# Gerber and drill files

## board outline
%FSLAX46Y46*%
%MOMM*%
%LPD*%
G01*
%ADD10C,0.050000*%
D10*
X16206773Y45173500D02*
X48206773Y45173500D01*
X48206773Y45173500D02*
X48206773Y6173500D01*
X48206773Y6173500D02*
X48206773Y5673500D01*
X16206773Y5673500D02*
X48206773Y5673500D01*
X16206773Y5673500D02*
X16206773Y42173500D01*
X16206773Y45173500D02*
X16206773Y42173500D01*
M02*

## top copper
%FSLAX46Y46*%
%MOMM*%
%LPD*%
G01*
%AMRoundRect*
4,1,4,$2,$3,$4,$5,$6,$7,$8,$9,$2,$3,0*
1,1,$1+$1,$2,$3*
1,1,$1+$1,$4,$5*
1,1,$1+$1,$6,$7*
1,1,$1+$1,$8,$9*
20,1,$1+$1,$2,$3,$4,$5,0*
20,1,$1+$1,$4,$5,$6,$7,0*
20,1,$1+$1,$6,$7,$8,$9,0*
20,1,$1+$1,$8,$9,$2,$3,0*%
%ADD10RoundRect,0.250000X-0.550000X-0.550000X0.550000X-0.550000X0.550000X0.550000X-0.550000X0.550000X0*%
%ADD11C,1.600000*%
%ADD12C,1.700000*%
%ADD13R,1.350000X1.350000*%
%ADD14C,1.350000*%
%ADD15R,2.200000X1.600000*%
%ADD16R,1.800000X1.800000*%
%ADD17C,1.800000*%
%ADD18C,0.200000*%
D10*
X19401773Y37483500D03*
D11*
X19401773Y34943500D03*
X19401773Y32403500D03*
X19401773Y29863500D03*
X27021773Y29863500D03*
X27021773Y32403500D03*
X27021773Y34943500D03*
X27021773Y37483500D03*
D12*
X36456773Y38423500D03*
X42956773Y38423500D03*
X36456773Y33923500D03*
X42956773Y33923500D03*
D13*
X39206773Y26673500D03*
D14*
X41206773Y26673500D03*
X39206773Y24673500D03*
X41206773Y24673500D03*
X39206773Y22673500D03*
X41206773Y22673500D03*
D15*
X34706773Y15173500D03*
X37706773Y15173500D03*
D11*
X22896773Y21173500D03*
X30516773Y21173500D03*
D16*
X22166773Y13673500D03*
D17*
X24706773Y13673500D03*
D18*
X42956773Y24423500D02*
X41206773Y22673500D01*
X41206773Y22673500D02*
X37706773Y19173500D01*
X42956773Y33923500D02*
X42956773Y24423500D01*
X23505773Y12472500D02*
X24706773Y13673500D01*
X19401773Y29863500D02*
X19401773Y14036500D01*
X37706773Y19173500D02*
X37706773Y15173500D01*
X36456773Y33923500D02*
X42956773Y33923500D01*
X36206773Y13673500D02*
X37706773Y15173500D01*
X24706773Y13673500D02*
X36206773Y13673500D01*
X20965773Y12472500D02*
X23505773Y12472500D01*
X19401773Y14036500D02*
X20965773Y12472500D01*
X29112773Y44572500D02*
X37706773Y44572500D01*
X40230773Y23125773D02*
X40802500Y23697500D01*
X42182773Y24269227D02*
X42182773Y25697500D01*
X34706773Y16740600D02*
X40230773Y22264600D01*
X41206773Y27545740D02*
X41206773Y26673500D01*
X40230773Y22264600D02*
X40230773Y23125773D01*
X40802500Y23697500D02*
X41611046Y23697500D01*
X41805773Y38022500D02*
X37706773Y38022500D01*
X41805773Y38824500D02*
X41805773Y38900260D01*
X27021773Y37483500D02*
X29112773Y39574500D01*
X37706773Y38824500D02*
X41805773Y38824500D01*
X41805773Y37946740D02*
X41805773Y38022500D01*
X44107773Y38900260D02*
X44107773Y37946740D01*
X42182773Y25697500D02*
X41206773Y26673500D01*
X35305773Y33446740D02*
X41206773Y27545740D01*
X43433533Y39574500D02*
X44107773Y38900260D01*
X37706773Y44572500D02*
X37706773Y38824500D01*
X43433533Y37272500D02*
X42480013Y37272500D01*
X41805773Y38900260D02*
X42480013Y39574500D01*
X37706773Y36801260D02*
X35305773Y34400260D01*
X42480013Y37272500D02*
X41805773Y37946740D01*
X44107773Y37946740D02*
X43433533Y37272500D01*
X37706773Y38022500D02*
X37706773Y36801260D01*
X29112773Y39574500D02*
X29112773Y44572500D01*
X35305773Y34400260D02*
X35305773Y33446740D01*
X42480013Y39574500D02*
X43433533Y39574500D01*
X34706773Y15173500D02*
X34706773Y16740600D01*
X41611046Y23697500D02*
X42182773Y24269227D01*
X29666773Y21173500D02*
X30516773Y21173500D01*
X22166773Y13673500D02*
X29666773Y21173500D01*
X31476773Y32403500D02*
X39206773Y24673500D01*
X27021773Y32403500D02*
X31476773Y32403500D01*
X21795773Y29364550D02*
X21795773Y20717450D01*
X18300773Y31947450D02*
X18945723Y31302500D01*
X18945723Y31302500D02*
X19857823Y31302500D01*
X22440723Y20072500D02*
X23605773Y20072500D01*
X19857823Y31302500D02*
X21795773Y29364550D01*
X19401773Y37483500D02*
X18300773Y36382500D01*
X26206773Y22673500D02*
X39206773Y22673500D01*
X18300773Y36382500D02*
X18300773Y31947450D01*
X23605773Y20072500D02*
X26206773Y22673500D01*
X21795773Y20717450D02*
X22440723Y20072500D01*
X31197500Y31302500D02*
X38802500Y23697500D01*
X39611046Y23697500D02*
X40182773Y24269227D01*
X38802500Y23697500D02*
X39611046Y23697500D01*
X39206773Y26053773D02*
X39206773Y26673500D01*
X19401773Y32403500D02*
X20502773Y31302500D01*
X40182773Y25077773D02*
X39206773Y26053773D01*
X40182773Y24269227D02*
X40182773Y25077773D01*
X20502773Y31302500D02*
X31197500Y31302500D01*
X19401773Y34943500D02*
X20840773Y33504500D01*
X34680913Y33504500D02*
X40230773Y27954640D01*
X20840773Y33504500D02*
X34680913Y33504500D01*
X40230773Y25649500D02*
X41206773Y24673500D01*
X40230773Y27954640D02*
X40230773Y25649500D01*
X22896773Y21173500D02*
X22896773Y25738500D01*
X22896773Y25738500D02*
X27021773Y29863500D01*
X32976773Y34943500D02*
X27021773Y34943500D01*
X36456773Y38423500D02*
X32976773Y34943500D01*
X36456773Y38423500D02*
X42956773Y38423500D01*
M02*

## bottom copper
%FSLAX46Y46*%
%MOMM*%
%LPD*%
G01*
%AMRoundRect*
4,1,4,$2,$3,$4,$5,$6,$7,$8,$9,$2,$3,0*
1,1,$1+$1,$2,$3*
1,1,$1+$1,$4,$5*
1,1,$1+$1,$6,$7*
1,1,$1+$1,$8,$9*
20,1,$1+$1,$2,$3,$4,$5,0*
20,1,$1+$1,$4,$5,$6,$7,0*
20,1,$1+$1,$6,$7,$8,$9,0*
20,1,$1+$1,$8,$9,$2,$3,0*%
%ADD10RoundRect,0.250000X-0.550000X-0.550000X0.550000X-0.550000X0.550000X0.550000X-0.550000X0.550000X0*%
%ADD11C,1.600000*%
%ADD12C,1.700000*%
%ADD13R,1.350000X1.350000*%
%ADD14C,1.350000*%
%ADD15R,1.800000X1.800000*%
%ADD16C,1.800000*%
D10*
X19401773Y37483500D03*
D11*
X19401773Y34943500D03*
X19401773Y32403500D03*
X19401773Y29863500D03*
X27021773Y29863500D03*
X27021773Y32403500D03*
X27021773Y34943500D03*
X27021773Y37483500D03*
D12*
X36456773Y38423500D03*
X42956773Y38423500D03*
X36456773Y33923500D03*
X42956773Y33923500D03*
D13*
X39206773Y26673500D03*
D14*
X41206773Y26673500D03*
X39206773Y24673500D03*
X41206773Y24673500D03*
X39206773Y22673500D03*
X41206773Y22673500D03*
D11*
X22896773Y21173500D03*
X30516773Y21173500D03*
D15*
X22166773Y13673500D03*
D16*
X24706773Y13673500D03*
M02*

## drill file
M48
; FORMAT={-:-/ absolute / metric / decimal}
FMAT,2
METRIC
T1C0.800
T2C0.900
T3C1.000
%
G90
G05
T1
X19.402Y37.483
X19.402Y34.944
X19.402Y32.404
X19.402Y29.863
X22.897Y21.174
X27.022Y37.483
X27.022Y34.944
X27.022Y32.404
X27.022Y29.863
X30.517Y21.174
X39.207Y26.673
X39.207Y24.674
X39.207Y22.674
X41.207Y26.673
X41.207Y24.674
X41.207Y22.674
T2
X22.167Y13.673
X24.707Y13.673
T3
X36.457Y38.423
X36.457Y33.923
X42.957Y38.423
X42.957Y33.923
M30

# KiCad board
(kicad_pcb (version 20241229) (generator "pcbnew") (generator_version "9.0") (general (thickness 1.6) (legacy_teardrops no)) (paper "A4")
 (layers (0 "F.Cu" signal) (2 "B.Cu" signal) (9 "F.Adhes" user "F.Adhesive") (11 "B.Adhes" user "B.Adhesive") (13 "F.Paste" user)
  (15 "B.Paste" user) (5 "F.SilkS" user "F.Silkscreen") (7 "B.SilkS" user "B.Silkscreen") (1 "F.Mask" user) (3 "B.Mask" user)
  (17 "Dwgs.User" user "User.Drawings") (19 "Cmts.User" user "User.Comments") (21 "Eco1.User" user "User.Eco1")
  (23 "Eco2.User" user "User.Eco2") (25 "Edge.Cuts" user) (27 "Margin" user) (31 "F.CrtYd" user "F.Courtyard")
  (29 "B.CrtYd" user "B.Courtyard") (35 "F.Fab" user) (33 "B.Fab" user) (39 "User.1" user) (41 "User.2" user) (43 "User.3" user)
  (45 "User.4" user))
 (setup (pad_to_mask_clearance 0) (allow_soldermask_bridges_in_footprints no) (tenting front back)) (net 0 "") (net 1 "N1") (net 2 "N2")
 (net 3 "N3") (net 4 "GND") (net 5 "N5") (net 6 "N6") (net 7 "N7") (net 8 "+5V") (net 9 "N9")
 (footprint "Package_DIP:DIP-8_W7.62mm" (layer "F.Cu") (at 19.401773 -37.4835)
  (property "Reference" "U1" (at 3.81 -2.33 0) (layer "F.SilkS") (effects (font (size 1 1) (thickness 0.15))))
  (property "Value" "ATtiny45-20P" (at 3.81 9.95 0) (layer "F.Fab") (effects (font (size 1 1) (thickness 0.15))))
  (pad "1" thru_hole roundrect (at 0 0) (size 1.6 1.6) (drill 0.8) (layers "*.Cu" "*.Mask") (remove_unused_layers no)
   (roundrect_rratio 0.15625) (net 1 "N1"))
  (pad "2" thru_hole circle (at 0 2.54) (size 1.6 1.6) (drill 0.8) (layers "*.Cu" "*.Mask") (remove_unused_layers no) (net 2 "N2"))
  (pad "3" thru_hole circle (at 0 5.08) (size 1.6 1.6) (drill 0.8) (layers "*.Cu" "*.Mask") (remove_unused_layers no) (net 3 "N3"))
  (pad "4" thru_hole circle (at 0 7.62) (size 1.6 1.6) (drill 0.8) (layers "*.Cu" "*.Mask") (remove_unused_layers no) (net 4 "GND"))
  (pad "5" thru_hole circle (at 7.62 7.62) (size 1.6 1.6) (drill 0.8) (layers "*.Cu" "*.Mask") (remove_unused_layers no) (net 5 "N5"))
  (pad "6" thru_hole circle (at 7.62 5.08) (size 1.6 1.6) (drill 0.8) (layers "*.Cu" "*.Mask") (remove_unused_layers no) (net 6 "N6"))
  (pad "7" thru_hole circle (at 7.62 2.54) (size 1.6 1.6) (drill 0.8) (layers "*.Cu" "*.Mask") (remove_unused_layers no) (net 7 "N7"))
  (pad "8" thru_hole circle (at 7.62 0) (size 1.6 1.6) (drill 0.8) (layers "*.Cu" "*.Mask") (remove_unused_layers no) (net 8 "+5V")))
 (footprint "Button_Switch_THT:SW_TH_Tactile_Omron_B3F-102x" (layer "F.Cu") (at 36.456773 -38.4235)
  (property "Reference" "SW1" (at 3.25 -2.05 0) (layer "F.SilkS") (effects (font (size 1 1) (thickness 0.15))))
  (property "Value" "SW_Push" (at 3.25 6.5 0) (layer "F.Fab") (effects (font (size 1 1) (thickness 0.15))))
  (pad "1" thru_hole circle (at 0 0) (size 1.7 1.7) (drill 1) (layers "*.Cu" "*.Mask") (remove_unused_layers no) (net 7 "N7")
   (thermal_bridge_angle 90))
  (pad "1" thru_hole circle (at 6.5 0) (size 1.7 1.7) (drill 1) (layers "*.Cu" "*.Mask") (remove_unused_layers no) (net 7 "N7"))
  (pad "2" thru_hole circle (at 0 4.5) (size 1.7 1.7) (drill 1) (layers "*.Cu" "*.Mask") (remove_unused_layers no) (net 4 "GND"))
  (pad "2" thru_hole circle (at 6.5 4.5) (size 1.7 1.7) (drill 1) (layers "*.Cu" "*.Mask") (remove_unused_layers no) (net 4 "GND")))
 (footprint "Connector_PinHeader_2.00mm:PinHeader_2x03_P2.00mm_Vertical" (layer "F.Cu") (at 39.206773 -26.6735)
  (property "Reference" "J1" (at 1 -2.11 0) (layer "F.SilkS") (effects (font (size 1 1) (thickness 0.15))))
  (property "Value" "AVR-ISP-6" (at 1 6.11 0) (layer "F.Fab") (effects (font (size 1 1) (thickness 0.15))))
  (pad "1" thru_hole rect (at 0 0) (size 1.35 1.35) (drill 0.8) (layers "*.Cu" "*.Mask") (remove_unused_layers no) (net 3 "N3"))
  (pad "2" thru_hole circle (at 2 0) (size 1.35 1.35) (drill 0.8) (layers "*.Cu" "*.Mask") (remove_unused_layers no) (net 8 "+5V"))
  (pad "3" thru_hole circle (at 0 2) (size 1.35 1.35) (drill 0.8) (layers "*.Cu" "*.Mask") (remove_unused_layers no) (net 6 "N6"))
  (pad "4" thru_hole circle (at 2 2) (size 1.35 1.35) (drill 0.8) (layers "*.Cu" "*.Mask") (remove_unused_layers no) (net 2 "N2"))
  (pad "5" thru_hole circle (at 0 4) (size 1.35 1.35) (drill 0.8) (layers "*.Cu" "*.Mask") (remove_unused_layers no) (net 1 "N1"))
  (pad "6" thru_hole circle (at 2 4) (size 1.35 1.35) (drill 0.8) (layers "*.Cu" "*.Mask") (remove_unused_layers no) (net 4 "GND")))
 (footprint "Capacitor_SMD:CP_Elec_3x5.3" (layer "F.Cu") (at 36.206773 -15.1735)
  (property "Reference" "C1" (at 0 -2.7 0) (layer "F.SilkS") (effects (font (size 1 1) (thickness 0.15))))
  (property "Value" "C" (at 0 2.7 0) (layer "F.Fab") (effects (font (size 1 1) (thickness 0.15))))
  (pad "1" smd rect (at -1.5 0) (size 2.2 1.6) (layers "F.Cu" "F.Mask" "F.Paste") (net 8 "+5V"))
  (pad "2" smd rect (at 1.5 0) (size 2.2 1.6) (layers "F.Cu" "F.Mask" "F.Paste") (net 4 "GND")))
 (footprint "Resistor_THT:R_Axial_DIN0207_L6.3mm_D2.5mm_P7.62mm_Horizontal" (layer "F.Cu") (at 22.896773 -21.1735)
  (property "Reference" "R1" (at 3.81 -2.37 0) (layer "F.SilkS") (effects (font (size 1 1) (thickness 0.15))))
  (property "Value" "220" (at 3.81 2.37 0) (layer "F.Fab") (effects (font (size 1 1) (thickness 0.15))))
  (pad "1" thru_hole circle (at 0 0) (size 1.6 1.6) (drill 0.8) (layers "*.Cu" "*.Mask") (remove_unused_layers no) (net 5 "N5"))
  (pad "2" thru_hole circle (at 7.62 0) (size 1.6 1.6) (drill 0.8) (layers "*.Cu" "*.Mask") (remove_unused_layers no) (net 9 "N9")))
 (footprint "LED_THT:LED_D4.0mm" (layer "F.Cu") (at 22.166773 -13.6735)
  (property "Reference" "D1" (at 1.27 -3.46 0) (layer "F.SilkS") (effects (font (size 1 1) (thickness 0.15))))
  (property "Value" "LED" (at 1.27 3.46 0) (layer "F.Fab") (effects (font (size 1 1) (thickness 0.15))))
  (pad "1" thru_hole rect (at 0 0) (size 1.8 1.8) (drill 0.9) (layers "*.Cu" "*.Mask") (remove_unused_layers no) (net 9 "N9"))
  (pad "2" thru_hole circle (at 2.54 0) (size 1.8 1.8) (drill 0.9) (layers "*.Cu" "*.Mask") (remove_unused_layers no) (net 4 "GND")))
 (gr_line (start 16.206773 -45.1735) (end 48.206773 -45.1735) (stroke (width 0.05) (type default)) (layer "Edge.Cuts"))
 (gr_line (start 48.206773 -45.1735) (end 48.206773 -6.1735) (stroke (width 0.05) (type default)) (layer "Edge.Cuts"))
 (gr_line (start 48.206773 -6.1735) (end 48.206773 -5.6735) (stroke (width 0.05) (type default)) (layer "Edge.Cuts"))
 (gr_line (start 16.206773 -5.6735) (end 48.206773 -5.6735) (stroke (width 0.05) (type default)) (layer "Edge.Cuts"))
 (gr_line (start 16.206773 -5.6735) (end 16.206773 -42.1735) (stroke (width 0.05) (type default)) (layer "Edge.Cuts"))
 (gr_line (start 16.206773 -45.1735) (end 16.206773 -42.1735) (stroke (width 0.05) (type default)) (layer "Edge.Cuts"))
 (segment (start 42.956773 -24.4235) (end 41.206773 -22.6735) (width 0.2) (layer "F.Cu") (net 4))
 (segment (start 41.206773 -22.6735) (end 37.706773 -19.1735) (width 0.2) (layer "F.Cu") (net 4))
 (segment (start 42.956773 -33.9235) (end 42.956773 -24.4235) (width 0.2) (layer "F.Cu") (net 4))
 (segment (start 23.505773 -12.4725) (end 24.706773 -13.6735) (width 0.2) (layer "F.Cu") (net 4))
 (segment (start 19.401773 -29.8635) (end 19.401773 -14.0365) (width 0.2) (layer "F.Cu") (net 4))
 (segment (start 37.706773 -19.1735) (end 37.706773 -15.1735) (width 0.2) (layer "F.Cu") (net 4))
 (segment (start 36.456773 -33.9235) (end 42.956773 -33.9235) (width 0.2) (layer "F.Cu") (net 4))
 (segment (start 36.206773 -13.6735) (end 37.706773 -15.1735) (width 0.2) (layer "F.Cu") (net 4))
 (segment (start 24.706773 -13.6735) (end 36.206773 -13.6735) (width 0.2) (layer "F.Cu") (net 4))
 (segment (start 20.965773 -12.4725) (end 23.505773 -12.4725) (width 0.2) (layer "F.Cu") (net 4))
 (segment (start 19.401773 -14.0365) (end 20.965773 -12.4725) (width 0.2) (layer "F.Cu") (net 4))
 (segment (start 29.112773 -44.5725) (end 37.706773 -44.5725) (width 0.2) (layer "F.Cu") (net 8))
 (segment (start 40.230773 -23.125773) (end 40.8025 -23.6975) (width 0.2) (layer "F.Cu") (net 8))
 (segment (start 42.182773 -24.269227) (end 42.182773 -25.6975) (width 0.2) (layer "F.Cu") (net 8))
 (segment (start 34.706773 -16.7406) (end 40.230773 -22.2646) (width 0.2) (layer "F.Cu") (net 8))
 (segment (start 41.206773 -27.54574) (end 41.206773 -26.6735) (width 0.2) (layer "F.Cu") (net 8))
 (segment (start 40.230773 -22.2646) (end 40.230773 -23.125773) (width 0.2) (layer "F.Cu") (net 8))
 (segment (start 40.8025 -23.6975) (end 41.611046 -23.6975) (width 0.2) (layer "F.Cu") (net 8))
 (segment (start 41.805773 -38.0225) (end 37.706773 -38.0225) (width 0.2) (layer "F.Cu") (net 8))
 (segment (start 41.805773 -38.8245) (end 41.805773 -38.90026) (width 0.2) (layer "F.Cu") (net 8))
 (segment (start 27.021773 -37.4835) (end 29.112773 -39.5745) (width 0.2) (layer "F.Cu") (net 8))
 (segment (start 37.706773 -38.8245) (end 41.805773 -38.8245) (width 0.2) (layer "F.Cu") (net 8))
 (segment (start 41.805773 -37.94674) (end 41.805773 -38.0225) (width 0.2) (layer "F.Cu") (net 8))
 (segment (start 44.107773 -38.90026) (end 44.107773 -37.94674) (width 0.2) (layer "F.Cu") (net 8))
 (segment (start 42.182773 -25.6975) (end 41.206773 -26.6735) (width 0.2) (layer "F.Cu") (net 8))
 (segment (start 35.305773 -33.44674) (end 41.206773 -27.54574) (width 0.2) (layer "F.Cu") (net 8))
 (segment (start 43.433533 -39.5745) (end 44.107773 -38.90026) (width 0.2) (layer "F.Cu") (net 8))
 (segment (start 37.706773 -44.5725) (end 37.706773 -38.8245) (width 0.2) (layer "F.Cu") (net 8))
 (segment (start 43.433533 -37.2725) (end 42.480013 -37.2725) (width 0.2) (layer "F.Cu") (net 8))
 (segment (start 41.805773 -38.90026) (end 42.480013 -39.5745) (width 0.2) (layer "F.Cu") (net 8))
 (segment (start 37.706773 -36.80126) (end 35.305773 -34.40026) (width 0.2) (layer "F.Cu") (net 8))
 (segment (start 42.480013 -37.2725) (end 41.805773 -37.94674) (width 0.2) (layer "F.Cu") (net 8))
 (segment (start 44.107773 -37.94674) (end 43.433533 -37.2725) (width 0.2) (layer "F.Cu") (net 8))
 (segment (start 37.706773 -38.0225) (end 37.706773 -36.80126) (width 0.2) (layer "F.Cu") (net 8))
 (segment (start 29.112773 -39.5745) (end 29.112773 -44.5725) (width 0.2) (layer "F.Cu") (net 8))
 (segment (start 35.305773 -34.40026) (end 35.305773 -33.44674) (width 0.2) (layer "F.Cu") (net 8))
 (segment (start 42.480013 -39.5745) (end 43.433533 -39.5745) (width 0.2) (layer "F.Cu") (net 8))
 (segment (start 34.706773 -15.1735) (end 34.706773 -16.7406) (width 0.2) (layer "F.Cu") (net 8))
 (segment (start 41.611046 -23.6975) (end 42.182773 -24.269227) (width 0.2) (layer "F.Cu") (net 8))
 (segment (start 29.666773 -21.1735) (end 30.516773 -21.1735) (width 0.2) (layer "F.Cu") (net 9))
 (segment (start 22.166773 -13.6735) (end 29.666773 -21.1735) (width 0.2) (layer "F.Cu") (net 9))
 (segment (start 31.476773 -32.4035) (end 39.206773 -24.6735) (width 0.2) (layer "F.Cu") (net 6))
 (segment (start 27.021773 -32.4035) (end 31.476773 -32.4035) (width 0.2) (layer "F.Cu") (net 6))
 (segment (start 21.795773 -29.36455) (end 21.795773 -20.71745) (width 0.2) (layer "F.Cu") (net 1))
 (segment (start 18.300773 -31.94745) (end 18.945723 -31.3025) (width 0.2) (layer "F.Cu") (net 1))
 (segment (start 18.945723 -31.3025) (end 19.857823 -31.3025) (width 0.2) (layer "F.Cu") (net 1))
 (segment (start 22.440723 -20.0725) (end 23.605773 -20.0725) (width 0.2) (layer "F.Cu") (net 1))
 (segment (start 19.857823 -31.3025) (end 21.795773 -29.36455) (width 0.2) (layer "F.Cu") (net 1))
 (segment (start 19.401773 -37.4835) (end 18.300773 -36.3825) (width 0.2) (layer "F.Cu") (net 1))
 (segment (start 26.206773 -22.6735) (end 39.206773 -22.6735) (width 0.2) (layer "F.Cu") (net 1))
 (segment (start 18.300773 -36.3825) (end 18.300773 -31.94745) (width 0.2) (layer "F.Cu") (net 1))
 (segment (start 23.605773 -20.0725) (end 26.206773 -22.6735) (width 0.2) (layer "F.Cu") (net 1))
 (segment (start 21.795773 -20.71745) (end 22.440723 -20.0725) (width 0.2) (layer "F.Cu") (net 1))
 (segment (start 31.1975 -31.3025) (end 38.8025 -23.6975) (width 0.2) (layer "F.Cu") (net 3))
 (segment (start 39.611046 -23.6975) (end 40.182773 -24.269227) (width 0.2) (layer "F.Cu") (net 3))
 (segment (start 38.8025 -23.6975) (end 39.611046 -23.6975) (width 0.2) (layer "F.Cu") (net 3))
 (segment (start 39.206773 -26.053773) (end 39.206773 -26.6735) (width 0.2) (layer "F.Cu") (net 3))
 (segment (start 19.401773 -32.4035) (end 20.502773 -31.3025) (width 0.2) (layer "F.Cu") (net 3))
 (segment (start 40.182773 -25.077773) (end 39.206773 -26.053773) (width 0.2) (layer "F.Cu") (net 3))
 (segment (start 40.182773 -24.269227) (end 40.182773 -25.077773) (width 0.2) (layer "F.Cu") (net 3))
 (segment (start 20.502773 -31.3025) (end 31.1975 -31.3025) (width 0.2) (layer "F.Cu") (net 3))
 (segment (start 19.401773 -34.9435) (end 20.840773 -33.5045) (width 0.2) (layer "F.Cu") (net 2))
 (segment (start 34.680913 -33.5045) (end 40.230773 -27.95464) (width 0.2) (layer "F.Cu") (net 2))
 (segment (start 20.840773 -33.5045) (end 34.680913 -33.5045) (width 0.2) (layer "F.Cu") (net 2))
 (segment (start 40.230773 -25.6495) (end 41.206773 -24.6735) (width 0.2) (layer "F.Cu") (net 2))
 (segment (start 40.230773 -27.95464) (end 40.230773 -25.6495) (width 0.2) (layer "F.Cu") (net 2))
 (segment (start 22.896773 -21.1735) (end 22.896773 -25.7385) (width 0.2) (layer "F.Cu") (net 5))
 (segment (start 22.896773 -25.7385) (end 27.021773 -29.8635) (width 0.2) (layer "F.Cu") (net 5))
 (segment (start 32.976773 -34.9435) (end 27.021773 -34.9435) (width 0.2) (layer "F.Cu") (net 7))
 (segment (start 36.456773 -38.4235) (end 32.976773 -34.9435) (width 0.2) (layer "F.Cu") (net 7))
 (segment (start 36.456773 -38.4235) (end 42.956773 -38.4235) (width 0.2) (layer "F.Cu") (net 7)))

